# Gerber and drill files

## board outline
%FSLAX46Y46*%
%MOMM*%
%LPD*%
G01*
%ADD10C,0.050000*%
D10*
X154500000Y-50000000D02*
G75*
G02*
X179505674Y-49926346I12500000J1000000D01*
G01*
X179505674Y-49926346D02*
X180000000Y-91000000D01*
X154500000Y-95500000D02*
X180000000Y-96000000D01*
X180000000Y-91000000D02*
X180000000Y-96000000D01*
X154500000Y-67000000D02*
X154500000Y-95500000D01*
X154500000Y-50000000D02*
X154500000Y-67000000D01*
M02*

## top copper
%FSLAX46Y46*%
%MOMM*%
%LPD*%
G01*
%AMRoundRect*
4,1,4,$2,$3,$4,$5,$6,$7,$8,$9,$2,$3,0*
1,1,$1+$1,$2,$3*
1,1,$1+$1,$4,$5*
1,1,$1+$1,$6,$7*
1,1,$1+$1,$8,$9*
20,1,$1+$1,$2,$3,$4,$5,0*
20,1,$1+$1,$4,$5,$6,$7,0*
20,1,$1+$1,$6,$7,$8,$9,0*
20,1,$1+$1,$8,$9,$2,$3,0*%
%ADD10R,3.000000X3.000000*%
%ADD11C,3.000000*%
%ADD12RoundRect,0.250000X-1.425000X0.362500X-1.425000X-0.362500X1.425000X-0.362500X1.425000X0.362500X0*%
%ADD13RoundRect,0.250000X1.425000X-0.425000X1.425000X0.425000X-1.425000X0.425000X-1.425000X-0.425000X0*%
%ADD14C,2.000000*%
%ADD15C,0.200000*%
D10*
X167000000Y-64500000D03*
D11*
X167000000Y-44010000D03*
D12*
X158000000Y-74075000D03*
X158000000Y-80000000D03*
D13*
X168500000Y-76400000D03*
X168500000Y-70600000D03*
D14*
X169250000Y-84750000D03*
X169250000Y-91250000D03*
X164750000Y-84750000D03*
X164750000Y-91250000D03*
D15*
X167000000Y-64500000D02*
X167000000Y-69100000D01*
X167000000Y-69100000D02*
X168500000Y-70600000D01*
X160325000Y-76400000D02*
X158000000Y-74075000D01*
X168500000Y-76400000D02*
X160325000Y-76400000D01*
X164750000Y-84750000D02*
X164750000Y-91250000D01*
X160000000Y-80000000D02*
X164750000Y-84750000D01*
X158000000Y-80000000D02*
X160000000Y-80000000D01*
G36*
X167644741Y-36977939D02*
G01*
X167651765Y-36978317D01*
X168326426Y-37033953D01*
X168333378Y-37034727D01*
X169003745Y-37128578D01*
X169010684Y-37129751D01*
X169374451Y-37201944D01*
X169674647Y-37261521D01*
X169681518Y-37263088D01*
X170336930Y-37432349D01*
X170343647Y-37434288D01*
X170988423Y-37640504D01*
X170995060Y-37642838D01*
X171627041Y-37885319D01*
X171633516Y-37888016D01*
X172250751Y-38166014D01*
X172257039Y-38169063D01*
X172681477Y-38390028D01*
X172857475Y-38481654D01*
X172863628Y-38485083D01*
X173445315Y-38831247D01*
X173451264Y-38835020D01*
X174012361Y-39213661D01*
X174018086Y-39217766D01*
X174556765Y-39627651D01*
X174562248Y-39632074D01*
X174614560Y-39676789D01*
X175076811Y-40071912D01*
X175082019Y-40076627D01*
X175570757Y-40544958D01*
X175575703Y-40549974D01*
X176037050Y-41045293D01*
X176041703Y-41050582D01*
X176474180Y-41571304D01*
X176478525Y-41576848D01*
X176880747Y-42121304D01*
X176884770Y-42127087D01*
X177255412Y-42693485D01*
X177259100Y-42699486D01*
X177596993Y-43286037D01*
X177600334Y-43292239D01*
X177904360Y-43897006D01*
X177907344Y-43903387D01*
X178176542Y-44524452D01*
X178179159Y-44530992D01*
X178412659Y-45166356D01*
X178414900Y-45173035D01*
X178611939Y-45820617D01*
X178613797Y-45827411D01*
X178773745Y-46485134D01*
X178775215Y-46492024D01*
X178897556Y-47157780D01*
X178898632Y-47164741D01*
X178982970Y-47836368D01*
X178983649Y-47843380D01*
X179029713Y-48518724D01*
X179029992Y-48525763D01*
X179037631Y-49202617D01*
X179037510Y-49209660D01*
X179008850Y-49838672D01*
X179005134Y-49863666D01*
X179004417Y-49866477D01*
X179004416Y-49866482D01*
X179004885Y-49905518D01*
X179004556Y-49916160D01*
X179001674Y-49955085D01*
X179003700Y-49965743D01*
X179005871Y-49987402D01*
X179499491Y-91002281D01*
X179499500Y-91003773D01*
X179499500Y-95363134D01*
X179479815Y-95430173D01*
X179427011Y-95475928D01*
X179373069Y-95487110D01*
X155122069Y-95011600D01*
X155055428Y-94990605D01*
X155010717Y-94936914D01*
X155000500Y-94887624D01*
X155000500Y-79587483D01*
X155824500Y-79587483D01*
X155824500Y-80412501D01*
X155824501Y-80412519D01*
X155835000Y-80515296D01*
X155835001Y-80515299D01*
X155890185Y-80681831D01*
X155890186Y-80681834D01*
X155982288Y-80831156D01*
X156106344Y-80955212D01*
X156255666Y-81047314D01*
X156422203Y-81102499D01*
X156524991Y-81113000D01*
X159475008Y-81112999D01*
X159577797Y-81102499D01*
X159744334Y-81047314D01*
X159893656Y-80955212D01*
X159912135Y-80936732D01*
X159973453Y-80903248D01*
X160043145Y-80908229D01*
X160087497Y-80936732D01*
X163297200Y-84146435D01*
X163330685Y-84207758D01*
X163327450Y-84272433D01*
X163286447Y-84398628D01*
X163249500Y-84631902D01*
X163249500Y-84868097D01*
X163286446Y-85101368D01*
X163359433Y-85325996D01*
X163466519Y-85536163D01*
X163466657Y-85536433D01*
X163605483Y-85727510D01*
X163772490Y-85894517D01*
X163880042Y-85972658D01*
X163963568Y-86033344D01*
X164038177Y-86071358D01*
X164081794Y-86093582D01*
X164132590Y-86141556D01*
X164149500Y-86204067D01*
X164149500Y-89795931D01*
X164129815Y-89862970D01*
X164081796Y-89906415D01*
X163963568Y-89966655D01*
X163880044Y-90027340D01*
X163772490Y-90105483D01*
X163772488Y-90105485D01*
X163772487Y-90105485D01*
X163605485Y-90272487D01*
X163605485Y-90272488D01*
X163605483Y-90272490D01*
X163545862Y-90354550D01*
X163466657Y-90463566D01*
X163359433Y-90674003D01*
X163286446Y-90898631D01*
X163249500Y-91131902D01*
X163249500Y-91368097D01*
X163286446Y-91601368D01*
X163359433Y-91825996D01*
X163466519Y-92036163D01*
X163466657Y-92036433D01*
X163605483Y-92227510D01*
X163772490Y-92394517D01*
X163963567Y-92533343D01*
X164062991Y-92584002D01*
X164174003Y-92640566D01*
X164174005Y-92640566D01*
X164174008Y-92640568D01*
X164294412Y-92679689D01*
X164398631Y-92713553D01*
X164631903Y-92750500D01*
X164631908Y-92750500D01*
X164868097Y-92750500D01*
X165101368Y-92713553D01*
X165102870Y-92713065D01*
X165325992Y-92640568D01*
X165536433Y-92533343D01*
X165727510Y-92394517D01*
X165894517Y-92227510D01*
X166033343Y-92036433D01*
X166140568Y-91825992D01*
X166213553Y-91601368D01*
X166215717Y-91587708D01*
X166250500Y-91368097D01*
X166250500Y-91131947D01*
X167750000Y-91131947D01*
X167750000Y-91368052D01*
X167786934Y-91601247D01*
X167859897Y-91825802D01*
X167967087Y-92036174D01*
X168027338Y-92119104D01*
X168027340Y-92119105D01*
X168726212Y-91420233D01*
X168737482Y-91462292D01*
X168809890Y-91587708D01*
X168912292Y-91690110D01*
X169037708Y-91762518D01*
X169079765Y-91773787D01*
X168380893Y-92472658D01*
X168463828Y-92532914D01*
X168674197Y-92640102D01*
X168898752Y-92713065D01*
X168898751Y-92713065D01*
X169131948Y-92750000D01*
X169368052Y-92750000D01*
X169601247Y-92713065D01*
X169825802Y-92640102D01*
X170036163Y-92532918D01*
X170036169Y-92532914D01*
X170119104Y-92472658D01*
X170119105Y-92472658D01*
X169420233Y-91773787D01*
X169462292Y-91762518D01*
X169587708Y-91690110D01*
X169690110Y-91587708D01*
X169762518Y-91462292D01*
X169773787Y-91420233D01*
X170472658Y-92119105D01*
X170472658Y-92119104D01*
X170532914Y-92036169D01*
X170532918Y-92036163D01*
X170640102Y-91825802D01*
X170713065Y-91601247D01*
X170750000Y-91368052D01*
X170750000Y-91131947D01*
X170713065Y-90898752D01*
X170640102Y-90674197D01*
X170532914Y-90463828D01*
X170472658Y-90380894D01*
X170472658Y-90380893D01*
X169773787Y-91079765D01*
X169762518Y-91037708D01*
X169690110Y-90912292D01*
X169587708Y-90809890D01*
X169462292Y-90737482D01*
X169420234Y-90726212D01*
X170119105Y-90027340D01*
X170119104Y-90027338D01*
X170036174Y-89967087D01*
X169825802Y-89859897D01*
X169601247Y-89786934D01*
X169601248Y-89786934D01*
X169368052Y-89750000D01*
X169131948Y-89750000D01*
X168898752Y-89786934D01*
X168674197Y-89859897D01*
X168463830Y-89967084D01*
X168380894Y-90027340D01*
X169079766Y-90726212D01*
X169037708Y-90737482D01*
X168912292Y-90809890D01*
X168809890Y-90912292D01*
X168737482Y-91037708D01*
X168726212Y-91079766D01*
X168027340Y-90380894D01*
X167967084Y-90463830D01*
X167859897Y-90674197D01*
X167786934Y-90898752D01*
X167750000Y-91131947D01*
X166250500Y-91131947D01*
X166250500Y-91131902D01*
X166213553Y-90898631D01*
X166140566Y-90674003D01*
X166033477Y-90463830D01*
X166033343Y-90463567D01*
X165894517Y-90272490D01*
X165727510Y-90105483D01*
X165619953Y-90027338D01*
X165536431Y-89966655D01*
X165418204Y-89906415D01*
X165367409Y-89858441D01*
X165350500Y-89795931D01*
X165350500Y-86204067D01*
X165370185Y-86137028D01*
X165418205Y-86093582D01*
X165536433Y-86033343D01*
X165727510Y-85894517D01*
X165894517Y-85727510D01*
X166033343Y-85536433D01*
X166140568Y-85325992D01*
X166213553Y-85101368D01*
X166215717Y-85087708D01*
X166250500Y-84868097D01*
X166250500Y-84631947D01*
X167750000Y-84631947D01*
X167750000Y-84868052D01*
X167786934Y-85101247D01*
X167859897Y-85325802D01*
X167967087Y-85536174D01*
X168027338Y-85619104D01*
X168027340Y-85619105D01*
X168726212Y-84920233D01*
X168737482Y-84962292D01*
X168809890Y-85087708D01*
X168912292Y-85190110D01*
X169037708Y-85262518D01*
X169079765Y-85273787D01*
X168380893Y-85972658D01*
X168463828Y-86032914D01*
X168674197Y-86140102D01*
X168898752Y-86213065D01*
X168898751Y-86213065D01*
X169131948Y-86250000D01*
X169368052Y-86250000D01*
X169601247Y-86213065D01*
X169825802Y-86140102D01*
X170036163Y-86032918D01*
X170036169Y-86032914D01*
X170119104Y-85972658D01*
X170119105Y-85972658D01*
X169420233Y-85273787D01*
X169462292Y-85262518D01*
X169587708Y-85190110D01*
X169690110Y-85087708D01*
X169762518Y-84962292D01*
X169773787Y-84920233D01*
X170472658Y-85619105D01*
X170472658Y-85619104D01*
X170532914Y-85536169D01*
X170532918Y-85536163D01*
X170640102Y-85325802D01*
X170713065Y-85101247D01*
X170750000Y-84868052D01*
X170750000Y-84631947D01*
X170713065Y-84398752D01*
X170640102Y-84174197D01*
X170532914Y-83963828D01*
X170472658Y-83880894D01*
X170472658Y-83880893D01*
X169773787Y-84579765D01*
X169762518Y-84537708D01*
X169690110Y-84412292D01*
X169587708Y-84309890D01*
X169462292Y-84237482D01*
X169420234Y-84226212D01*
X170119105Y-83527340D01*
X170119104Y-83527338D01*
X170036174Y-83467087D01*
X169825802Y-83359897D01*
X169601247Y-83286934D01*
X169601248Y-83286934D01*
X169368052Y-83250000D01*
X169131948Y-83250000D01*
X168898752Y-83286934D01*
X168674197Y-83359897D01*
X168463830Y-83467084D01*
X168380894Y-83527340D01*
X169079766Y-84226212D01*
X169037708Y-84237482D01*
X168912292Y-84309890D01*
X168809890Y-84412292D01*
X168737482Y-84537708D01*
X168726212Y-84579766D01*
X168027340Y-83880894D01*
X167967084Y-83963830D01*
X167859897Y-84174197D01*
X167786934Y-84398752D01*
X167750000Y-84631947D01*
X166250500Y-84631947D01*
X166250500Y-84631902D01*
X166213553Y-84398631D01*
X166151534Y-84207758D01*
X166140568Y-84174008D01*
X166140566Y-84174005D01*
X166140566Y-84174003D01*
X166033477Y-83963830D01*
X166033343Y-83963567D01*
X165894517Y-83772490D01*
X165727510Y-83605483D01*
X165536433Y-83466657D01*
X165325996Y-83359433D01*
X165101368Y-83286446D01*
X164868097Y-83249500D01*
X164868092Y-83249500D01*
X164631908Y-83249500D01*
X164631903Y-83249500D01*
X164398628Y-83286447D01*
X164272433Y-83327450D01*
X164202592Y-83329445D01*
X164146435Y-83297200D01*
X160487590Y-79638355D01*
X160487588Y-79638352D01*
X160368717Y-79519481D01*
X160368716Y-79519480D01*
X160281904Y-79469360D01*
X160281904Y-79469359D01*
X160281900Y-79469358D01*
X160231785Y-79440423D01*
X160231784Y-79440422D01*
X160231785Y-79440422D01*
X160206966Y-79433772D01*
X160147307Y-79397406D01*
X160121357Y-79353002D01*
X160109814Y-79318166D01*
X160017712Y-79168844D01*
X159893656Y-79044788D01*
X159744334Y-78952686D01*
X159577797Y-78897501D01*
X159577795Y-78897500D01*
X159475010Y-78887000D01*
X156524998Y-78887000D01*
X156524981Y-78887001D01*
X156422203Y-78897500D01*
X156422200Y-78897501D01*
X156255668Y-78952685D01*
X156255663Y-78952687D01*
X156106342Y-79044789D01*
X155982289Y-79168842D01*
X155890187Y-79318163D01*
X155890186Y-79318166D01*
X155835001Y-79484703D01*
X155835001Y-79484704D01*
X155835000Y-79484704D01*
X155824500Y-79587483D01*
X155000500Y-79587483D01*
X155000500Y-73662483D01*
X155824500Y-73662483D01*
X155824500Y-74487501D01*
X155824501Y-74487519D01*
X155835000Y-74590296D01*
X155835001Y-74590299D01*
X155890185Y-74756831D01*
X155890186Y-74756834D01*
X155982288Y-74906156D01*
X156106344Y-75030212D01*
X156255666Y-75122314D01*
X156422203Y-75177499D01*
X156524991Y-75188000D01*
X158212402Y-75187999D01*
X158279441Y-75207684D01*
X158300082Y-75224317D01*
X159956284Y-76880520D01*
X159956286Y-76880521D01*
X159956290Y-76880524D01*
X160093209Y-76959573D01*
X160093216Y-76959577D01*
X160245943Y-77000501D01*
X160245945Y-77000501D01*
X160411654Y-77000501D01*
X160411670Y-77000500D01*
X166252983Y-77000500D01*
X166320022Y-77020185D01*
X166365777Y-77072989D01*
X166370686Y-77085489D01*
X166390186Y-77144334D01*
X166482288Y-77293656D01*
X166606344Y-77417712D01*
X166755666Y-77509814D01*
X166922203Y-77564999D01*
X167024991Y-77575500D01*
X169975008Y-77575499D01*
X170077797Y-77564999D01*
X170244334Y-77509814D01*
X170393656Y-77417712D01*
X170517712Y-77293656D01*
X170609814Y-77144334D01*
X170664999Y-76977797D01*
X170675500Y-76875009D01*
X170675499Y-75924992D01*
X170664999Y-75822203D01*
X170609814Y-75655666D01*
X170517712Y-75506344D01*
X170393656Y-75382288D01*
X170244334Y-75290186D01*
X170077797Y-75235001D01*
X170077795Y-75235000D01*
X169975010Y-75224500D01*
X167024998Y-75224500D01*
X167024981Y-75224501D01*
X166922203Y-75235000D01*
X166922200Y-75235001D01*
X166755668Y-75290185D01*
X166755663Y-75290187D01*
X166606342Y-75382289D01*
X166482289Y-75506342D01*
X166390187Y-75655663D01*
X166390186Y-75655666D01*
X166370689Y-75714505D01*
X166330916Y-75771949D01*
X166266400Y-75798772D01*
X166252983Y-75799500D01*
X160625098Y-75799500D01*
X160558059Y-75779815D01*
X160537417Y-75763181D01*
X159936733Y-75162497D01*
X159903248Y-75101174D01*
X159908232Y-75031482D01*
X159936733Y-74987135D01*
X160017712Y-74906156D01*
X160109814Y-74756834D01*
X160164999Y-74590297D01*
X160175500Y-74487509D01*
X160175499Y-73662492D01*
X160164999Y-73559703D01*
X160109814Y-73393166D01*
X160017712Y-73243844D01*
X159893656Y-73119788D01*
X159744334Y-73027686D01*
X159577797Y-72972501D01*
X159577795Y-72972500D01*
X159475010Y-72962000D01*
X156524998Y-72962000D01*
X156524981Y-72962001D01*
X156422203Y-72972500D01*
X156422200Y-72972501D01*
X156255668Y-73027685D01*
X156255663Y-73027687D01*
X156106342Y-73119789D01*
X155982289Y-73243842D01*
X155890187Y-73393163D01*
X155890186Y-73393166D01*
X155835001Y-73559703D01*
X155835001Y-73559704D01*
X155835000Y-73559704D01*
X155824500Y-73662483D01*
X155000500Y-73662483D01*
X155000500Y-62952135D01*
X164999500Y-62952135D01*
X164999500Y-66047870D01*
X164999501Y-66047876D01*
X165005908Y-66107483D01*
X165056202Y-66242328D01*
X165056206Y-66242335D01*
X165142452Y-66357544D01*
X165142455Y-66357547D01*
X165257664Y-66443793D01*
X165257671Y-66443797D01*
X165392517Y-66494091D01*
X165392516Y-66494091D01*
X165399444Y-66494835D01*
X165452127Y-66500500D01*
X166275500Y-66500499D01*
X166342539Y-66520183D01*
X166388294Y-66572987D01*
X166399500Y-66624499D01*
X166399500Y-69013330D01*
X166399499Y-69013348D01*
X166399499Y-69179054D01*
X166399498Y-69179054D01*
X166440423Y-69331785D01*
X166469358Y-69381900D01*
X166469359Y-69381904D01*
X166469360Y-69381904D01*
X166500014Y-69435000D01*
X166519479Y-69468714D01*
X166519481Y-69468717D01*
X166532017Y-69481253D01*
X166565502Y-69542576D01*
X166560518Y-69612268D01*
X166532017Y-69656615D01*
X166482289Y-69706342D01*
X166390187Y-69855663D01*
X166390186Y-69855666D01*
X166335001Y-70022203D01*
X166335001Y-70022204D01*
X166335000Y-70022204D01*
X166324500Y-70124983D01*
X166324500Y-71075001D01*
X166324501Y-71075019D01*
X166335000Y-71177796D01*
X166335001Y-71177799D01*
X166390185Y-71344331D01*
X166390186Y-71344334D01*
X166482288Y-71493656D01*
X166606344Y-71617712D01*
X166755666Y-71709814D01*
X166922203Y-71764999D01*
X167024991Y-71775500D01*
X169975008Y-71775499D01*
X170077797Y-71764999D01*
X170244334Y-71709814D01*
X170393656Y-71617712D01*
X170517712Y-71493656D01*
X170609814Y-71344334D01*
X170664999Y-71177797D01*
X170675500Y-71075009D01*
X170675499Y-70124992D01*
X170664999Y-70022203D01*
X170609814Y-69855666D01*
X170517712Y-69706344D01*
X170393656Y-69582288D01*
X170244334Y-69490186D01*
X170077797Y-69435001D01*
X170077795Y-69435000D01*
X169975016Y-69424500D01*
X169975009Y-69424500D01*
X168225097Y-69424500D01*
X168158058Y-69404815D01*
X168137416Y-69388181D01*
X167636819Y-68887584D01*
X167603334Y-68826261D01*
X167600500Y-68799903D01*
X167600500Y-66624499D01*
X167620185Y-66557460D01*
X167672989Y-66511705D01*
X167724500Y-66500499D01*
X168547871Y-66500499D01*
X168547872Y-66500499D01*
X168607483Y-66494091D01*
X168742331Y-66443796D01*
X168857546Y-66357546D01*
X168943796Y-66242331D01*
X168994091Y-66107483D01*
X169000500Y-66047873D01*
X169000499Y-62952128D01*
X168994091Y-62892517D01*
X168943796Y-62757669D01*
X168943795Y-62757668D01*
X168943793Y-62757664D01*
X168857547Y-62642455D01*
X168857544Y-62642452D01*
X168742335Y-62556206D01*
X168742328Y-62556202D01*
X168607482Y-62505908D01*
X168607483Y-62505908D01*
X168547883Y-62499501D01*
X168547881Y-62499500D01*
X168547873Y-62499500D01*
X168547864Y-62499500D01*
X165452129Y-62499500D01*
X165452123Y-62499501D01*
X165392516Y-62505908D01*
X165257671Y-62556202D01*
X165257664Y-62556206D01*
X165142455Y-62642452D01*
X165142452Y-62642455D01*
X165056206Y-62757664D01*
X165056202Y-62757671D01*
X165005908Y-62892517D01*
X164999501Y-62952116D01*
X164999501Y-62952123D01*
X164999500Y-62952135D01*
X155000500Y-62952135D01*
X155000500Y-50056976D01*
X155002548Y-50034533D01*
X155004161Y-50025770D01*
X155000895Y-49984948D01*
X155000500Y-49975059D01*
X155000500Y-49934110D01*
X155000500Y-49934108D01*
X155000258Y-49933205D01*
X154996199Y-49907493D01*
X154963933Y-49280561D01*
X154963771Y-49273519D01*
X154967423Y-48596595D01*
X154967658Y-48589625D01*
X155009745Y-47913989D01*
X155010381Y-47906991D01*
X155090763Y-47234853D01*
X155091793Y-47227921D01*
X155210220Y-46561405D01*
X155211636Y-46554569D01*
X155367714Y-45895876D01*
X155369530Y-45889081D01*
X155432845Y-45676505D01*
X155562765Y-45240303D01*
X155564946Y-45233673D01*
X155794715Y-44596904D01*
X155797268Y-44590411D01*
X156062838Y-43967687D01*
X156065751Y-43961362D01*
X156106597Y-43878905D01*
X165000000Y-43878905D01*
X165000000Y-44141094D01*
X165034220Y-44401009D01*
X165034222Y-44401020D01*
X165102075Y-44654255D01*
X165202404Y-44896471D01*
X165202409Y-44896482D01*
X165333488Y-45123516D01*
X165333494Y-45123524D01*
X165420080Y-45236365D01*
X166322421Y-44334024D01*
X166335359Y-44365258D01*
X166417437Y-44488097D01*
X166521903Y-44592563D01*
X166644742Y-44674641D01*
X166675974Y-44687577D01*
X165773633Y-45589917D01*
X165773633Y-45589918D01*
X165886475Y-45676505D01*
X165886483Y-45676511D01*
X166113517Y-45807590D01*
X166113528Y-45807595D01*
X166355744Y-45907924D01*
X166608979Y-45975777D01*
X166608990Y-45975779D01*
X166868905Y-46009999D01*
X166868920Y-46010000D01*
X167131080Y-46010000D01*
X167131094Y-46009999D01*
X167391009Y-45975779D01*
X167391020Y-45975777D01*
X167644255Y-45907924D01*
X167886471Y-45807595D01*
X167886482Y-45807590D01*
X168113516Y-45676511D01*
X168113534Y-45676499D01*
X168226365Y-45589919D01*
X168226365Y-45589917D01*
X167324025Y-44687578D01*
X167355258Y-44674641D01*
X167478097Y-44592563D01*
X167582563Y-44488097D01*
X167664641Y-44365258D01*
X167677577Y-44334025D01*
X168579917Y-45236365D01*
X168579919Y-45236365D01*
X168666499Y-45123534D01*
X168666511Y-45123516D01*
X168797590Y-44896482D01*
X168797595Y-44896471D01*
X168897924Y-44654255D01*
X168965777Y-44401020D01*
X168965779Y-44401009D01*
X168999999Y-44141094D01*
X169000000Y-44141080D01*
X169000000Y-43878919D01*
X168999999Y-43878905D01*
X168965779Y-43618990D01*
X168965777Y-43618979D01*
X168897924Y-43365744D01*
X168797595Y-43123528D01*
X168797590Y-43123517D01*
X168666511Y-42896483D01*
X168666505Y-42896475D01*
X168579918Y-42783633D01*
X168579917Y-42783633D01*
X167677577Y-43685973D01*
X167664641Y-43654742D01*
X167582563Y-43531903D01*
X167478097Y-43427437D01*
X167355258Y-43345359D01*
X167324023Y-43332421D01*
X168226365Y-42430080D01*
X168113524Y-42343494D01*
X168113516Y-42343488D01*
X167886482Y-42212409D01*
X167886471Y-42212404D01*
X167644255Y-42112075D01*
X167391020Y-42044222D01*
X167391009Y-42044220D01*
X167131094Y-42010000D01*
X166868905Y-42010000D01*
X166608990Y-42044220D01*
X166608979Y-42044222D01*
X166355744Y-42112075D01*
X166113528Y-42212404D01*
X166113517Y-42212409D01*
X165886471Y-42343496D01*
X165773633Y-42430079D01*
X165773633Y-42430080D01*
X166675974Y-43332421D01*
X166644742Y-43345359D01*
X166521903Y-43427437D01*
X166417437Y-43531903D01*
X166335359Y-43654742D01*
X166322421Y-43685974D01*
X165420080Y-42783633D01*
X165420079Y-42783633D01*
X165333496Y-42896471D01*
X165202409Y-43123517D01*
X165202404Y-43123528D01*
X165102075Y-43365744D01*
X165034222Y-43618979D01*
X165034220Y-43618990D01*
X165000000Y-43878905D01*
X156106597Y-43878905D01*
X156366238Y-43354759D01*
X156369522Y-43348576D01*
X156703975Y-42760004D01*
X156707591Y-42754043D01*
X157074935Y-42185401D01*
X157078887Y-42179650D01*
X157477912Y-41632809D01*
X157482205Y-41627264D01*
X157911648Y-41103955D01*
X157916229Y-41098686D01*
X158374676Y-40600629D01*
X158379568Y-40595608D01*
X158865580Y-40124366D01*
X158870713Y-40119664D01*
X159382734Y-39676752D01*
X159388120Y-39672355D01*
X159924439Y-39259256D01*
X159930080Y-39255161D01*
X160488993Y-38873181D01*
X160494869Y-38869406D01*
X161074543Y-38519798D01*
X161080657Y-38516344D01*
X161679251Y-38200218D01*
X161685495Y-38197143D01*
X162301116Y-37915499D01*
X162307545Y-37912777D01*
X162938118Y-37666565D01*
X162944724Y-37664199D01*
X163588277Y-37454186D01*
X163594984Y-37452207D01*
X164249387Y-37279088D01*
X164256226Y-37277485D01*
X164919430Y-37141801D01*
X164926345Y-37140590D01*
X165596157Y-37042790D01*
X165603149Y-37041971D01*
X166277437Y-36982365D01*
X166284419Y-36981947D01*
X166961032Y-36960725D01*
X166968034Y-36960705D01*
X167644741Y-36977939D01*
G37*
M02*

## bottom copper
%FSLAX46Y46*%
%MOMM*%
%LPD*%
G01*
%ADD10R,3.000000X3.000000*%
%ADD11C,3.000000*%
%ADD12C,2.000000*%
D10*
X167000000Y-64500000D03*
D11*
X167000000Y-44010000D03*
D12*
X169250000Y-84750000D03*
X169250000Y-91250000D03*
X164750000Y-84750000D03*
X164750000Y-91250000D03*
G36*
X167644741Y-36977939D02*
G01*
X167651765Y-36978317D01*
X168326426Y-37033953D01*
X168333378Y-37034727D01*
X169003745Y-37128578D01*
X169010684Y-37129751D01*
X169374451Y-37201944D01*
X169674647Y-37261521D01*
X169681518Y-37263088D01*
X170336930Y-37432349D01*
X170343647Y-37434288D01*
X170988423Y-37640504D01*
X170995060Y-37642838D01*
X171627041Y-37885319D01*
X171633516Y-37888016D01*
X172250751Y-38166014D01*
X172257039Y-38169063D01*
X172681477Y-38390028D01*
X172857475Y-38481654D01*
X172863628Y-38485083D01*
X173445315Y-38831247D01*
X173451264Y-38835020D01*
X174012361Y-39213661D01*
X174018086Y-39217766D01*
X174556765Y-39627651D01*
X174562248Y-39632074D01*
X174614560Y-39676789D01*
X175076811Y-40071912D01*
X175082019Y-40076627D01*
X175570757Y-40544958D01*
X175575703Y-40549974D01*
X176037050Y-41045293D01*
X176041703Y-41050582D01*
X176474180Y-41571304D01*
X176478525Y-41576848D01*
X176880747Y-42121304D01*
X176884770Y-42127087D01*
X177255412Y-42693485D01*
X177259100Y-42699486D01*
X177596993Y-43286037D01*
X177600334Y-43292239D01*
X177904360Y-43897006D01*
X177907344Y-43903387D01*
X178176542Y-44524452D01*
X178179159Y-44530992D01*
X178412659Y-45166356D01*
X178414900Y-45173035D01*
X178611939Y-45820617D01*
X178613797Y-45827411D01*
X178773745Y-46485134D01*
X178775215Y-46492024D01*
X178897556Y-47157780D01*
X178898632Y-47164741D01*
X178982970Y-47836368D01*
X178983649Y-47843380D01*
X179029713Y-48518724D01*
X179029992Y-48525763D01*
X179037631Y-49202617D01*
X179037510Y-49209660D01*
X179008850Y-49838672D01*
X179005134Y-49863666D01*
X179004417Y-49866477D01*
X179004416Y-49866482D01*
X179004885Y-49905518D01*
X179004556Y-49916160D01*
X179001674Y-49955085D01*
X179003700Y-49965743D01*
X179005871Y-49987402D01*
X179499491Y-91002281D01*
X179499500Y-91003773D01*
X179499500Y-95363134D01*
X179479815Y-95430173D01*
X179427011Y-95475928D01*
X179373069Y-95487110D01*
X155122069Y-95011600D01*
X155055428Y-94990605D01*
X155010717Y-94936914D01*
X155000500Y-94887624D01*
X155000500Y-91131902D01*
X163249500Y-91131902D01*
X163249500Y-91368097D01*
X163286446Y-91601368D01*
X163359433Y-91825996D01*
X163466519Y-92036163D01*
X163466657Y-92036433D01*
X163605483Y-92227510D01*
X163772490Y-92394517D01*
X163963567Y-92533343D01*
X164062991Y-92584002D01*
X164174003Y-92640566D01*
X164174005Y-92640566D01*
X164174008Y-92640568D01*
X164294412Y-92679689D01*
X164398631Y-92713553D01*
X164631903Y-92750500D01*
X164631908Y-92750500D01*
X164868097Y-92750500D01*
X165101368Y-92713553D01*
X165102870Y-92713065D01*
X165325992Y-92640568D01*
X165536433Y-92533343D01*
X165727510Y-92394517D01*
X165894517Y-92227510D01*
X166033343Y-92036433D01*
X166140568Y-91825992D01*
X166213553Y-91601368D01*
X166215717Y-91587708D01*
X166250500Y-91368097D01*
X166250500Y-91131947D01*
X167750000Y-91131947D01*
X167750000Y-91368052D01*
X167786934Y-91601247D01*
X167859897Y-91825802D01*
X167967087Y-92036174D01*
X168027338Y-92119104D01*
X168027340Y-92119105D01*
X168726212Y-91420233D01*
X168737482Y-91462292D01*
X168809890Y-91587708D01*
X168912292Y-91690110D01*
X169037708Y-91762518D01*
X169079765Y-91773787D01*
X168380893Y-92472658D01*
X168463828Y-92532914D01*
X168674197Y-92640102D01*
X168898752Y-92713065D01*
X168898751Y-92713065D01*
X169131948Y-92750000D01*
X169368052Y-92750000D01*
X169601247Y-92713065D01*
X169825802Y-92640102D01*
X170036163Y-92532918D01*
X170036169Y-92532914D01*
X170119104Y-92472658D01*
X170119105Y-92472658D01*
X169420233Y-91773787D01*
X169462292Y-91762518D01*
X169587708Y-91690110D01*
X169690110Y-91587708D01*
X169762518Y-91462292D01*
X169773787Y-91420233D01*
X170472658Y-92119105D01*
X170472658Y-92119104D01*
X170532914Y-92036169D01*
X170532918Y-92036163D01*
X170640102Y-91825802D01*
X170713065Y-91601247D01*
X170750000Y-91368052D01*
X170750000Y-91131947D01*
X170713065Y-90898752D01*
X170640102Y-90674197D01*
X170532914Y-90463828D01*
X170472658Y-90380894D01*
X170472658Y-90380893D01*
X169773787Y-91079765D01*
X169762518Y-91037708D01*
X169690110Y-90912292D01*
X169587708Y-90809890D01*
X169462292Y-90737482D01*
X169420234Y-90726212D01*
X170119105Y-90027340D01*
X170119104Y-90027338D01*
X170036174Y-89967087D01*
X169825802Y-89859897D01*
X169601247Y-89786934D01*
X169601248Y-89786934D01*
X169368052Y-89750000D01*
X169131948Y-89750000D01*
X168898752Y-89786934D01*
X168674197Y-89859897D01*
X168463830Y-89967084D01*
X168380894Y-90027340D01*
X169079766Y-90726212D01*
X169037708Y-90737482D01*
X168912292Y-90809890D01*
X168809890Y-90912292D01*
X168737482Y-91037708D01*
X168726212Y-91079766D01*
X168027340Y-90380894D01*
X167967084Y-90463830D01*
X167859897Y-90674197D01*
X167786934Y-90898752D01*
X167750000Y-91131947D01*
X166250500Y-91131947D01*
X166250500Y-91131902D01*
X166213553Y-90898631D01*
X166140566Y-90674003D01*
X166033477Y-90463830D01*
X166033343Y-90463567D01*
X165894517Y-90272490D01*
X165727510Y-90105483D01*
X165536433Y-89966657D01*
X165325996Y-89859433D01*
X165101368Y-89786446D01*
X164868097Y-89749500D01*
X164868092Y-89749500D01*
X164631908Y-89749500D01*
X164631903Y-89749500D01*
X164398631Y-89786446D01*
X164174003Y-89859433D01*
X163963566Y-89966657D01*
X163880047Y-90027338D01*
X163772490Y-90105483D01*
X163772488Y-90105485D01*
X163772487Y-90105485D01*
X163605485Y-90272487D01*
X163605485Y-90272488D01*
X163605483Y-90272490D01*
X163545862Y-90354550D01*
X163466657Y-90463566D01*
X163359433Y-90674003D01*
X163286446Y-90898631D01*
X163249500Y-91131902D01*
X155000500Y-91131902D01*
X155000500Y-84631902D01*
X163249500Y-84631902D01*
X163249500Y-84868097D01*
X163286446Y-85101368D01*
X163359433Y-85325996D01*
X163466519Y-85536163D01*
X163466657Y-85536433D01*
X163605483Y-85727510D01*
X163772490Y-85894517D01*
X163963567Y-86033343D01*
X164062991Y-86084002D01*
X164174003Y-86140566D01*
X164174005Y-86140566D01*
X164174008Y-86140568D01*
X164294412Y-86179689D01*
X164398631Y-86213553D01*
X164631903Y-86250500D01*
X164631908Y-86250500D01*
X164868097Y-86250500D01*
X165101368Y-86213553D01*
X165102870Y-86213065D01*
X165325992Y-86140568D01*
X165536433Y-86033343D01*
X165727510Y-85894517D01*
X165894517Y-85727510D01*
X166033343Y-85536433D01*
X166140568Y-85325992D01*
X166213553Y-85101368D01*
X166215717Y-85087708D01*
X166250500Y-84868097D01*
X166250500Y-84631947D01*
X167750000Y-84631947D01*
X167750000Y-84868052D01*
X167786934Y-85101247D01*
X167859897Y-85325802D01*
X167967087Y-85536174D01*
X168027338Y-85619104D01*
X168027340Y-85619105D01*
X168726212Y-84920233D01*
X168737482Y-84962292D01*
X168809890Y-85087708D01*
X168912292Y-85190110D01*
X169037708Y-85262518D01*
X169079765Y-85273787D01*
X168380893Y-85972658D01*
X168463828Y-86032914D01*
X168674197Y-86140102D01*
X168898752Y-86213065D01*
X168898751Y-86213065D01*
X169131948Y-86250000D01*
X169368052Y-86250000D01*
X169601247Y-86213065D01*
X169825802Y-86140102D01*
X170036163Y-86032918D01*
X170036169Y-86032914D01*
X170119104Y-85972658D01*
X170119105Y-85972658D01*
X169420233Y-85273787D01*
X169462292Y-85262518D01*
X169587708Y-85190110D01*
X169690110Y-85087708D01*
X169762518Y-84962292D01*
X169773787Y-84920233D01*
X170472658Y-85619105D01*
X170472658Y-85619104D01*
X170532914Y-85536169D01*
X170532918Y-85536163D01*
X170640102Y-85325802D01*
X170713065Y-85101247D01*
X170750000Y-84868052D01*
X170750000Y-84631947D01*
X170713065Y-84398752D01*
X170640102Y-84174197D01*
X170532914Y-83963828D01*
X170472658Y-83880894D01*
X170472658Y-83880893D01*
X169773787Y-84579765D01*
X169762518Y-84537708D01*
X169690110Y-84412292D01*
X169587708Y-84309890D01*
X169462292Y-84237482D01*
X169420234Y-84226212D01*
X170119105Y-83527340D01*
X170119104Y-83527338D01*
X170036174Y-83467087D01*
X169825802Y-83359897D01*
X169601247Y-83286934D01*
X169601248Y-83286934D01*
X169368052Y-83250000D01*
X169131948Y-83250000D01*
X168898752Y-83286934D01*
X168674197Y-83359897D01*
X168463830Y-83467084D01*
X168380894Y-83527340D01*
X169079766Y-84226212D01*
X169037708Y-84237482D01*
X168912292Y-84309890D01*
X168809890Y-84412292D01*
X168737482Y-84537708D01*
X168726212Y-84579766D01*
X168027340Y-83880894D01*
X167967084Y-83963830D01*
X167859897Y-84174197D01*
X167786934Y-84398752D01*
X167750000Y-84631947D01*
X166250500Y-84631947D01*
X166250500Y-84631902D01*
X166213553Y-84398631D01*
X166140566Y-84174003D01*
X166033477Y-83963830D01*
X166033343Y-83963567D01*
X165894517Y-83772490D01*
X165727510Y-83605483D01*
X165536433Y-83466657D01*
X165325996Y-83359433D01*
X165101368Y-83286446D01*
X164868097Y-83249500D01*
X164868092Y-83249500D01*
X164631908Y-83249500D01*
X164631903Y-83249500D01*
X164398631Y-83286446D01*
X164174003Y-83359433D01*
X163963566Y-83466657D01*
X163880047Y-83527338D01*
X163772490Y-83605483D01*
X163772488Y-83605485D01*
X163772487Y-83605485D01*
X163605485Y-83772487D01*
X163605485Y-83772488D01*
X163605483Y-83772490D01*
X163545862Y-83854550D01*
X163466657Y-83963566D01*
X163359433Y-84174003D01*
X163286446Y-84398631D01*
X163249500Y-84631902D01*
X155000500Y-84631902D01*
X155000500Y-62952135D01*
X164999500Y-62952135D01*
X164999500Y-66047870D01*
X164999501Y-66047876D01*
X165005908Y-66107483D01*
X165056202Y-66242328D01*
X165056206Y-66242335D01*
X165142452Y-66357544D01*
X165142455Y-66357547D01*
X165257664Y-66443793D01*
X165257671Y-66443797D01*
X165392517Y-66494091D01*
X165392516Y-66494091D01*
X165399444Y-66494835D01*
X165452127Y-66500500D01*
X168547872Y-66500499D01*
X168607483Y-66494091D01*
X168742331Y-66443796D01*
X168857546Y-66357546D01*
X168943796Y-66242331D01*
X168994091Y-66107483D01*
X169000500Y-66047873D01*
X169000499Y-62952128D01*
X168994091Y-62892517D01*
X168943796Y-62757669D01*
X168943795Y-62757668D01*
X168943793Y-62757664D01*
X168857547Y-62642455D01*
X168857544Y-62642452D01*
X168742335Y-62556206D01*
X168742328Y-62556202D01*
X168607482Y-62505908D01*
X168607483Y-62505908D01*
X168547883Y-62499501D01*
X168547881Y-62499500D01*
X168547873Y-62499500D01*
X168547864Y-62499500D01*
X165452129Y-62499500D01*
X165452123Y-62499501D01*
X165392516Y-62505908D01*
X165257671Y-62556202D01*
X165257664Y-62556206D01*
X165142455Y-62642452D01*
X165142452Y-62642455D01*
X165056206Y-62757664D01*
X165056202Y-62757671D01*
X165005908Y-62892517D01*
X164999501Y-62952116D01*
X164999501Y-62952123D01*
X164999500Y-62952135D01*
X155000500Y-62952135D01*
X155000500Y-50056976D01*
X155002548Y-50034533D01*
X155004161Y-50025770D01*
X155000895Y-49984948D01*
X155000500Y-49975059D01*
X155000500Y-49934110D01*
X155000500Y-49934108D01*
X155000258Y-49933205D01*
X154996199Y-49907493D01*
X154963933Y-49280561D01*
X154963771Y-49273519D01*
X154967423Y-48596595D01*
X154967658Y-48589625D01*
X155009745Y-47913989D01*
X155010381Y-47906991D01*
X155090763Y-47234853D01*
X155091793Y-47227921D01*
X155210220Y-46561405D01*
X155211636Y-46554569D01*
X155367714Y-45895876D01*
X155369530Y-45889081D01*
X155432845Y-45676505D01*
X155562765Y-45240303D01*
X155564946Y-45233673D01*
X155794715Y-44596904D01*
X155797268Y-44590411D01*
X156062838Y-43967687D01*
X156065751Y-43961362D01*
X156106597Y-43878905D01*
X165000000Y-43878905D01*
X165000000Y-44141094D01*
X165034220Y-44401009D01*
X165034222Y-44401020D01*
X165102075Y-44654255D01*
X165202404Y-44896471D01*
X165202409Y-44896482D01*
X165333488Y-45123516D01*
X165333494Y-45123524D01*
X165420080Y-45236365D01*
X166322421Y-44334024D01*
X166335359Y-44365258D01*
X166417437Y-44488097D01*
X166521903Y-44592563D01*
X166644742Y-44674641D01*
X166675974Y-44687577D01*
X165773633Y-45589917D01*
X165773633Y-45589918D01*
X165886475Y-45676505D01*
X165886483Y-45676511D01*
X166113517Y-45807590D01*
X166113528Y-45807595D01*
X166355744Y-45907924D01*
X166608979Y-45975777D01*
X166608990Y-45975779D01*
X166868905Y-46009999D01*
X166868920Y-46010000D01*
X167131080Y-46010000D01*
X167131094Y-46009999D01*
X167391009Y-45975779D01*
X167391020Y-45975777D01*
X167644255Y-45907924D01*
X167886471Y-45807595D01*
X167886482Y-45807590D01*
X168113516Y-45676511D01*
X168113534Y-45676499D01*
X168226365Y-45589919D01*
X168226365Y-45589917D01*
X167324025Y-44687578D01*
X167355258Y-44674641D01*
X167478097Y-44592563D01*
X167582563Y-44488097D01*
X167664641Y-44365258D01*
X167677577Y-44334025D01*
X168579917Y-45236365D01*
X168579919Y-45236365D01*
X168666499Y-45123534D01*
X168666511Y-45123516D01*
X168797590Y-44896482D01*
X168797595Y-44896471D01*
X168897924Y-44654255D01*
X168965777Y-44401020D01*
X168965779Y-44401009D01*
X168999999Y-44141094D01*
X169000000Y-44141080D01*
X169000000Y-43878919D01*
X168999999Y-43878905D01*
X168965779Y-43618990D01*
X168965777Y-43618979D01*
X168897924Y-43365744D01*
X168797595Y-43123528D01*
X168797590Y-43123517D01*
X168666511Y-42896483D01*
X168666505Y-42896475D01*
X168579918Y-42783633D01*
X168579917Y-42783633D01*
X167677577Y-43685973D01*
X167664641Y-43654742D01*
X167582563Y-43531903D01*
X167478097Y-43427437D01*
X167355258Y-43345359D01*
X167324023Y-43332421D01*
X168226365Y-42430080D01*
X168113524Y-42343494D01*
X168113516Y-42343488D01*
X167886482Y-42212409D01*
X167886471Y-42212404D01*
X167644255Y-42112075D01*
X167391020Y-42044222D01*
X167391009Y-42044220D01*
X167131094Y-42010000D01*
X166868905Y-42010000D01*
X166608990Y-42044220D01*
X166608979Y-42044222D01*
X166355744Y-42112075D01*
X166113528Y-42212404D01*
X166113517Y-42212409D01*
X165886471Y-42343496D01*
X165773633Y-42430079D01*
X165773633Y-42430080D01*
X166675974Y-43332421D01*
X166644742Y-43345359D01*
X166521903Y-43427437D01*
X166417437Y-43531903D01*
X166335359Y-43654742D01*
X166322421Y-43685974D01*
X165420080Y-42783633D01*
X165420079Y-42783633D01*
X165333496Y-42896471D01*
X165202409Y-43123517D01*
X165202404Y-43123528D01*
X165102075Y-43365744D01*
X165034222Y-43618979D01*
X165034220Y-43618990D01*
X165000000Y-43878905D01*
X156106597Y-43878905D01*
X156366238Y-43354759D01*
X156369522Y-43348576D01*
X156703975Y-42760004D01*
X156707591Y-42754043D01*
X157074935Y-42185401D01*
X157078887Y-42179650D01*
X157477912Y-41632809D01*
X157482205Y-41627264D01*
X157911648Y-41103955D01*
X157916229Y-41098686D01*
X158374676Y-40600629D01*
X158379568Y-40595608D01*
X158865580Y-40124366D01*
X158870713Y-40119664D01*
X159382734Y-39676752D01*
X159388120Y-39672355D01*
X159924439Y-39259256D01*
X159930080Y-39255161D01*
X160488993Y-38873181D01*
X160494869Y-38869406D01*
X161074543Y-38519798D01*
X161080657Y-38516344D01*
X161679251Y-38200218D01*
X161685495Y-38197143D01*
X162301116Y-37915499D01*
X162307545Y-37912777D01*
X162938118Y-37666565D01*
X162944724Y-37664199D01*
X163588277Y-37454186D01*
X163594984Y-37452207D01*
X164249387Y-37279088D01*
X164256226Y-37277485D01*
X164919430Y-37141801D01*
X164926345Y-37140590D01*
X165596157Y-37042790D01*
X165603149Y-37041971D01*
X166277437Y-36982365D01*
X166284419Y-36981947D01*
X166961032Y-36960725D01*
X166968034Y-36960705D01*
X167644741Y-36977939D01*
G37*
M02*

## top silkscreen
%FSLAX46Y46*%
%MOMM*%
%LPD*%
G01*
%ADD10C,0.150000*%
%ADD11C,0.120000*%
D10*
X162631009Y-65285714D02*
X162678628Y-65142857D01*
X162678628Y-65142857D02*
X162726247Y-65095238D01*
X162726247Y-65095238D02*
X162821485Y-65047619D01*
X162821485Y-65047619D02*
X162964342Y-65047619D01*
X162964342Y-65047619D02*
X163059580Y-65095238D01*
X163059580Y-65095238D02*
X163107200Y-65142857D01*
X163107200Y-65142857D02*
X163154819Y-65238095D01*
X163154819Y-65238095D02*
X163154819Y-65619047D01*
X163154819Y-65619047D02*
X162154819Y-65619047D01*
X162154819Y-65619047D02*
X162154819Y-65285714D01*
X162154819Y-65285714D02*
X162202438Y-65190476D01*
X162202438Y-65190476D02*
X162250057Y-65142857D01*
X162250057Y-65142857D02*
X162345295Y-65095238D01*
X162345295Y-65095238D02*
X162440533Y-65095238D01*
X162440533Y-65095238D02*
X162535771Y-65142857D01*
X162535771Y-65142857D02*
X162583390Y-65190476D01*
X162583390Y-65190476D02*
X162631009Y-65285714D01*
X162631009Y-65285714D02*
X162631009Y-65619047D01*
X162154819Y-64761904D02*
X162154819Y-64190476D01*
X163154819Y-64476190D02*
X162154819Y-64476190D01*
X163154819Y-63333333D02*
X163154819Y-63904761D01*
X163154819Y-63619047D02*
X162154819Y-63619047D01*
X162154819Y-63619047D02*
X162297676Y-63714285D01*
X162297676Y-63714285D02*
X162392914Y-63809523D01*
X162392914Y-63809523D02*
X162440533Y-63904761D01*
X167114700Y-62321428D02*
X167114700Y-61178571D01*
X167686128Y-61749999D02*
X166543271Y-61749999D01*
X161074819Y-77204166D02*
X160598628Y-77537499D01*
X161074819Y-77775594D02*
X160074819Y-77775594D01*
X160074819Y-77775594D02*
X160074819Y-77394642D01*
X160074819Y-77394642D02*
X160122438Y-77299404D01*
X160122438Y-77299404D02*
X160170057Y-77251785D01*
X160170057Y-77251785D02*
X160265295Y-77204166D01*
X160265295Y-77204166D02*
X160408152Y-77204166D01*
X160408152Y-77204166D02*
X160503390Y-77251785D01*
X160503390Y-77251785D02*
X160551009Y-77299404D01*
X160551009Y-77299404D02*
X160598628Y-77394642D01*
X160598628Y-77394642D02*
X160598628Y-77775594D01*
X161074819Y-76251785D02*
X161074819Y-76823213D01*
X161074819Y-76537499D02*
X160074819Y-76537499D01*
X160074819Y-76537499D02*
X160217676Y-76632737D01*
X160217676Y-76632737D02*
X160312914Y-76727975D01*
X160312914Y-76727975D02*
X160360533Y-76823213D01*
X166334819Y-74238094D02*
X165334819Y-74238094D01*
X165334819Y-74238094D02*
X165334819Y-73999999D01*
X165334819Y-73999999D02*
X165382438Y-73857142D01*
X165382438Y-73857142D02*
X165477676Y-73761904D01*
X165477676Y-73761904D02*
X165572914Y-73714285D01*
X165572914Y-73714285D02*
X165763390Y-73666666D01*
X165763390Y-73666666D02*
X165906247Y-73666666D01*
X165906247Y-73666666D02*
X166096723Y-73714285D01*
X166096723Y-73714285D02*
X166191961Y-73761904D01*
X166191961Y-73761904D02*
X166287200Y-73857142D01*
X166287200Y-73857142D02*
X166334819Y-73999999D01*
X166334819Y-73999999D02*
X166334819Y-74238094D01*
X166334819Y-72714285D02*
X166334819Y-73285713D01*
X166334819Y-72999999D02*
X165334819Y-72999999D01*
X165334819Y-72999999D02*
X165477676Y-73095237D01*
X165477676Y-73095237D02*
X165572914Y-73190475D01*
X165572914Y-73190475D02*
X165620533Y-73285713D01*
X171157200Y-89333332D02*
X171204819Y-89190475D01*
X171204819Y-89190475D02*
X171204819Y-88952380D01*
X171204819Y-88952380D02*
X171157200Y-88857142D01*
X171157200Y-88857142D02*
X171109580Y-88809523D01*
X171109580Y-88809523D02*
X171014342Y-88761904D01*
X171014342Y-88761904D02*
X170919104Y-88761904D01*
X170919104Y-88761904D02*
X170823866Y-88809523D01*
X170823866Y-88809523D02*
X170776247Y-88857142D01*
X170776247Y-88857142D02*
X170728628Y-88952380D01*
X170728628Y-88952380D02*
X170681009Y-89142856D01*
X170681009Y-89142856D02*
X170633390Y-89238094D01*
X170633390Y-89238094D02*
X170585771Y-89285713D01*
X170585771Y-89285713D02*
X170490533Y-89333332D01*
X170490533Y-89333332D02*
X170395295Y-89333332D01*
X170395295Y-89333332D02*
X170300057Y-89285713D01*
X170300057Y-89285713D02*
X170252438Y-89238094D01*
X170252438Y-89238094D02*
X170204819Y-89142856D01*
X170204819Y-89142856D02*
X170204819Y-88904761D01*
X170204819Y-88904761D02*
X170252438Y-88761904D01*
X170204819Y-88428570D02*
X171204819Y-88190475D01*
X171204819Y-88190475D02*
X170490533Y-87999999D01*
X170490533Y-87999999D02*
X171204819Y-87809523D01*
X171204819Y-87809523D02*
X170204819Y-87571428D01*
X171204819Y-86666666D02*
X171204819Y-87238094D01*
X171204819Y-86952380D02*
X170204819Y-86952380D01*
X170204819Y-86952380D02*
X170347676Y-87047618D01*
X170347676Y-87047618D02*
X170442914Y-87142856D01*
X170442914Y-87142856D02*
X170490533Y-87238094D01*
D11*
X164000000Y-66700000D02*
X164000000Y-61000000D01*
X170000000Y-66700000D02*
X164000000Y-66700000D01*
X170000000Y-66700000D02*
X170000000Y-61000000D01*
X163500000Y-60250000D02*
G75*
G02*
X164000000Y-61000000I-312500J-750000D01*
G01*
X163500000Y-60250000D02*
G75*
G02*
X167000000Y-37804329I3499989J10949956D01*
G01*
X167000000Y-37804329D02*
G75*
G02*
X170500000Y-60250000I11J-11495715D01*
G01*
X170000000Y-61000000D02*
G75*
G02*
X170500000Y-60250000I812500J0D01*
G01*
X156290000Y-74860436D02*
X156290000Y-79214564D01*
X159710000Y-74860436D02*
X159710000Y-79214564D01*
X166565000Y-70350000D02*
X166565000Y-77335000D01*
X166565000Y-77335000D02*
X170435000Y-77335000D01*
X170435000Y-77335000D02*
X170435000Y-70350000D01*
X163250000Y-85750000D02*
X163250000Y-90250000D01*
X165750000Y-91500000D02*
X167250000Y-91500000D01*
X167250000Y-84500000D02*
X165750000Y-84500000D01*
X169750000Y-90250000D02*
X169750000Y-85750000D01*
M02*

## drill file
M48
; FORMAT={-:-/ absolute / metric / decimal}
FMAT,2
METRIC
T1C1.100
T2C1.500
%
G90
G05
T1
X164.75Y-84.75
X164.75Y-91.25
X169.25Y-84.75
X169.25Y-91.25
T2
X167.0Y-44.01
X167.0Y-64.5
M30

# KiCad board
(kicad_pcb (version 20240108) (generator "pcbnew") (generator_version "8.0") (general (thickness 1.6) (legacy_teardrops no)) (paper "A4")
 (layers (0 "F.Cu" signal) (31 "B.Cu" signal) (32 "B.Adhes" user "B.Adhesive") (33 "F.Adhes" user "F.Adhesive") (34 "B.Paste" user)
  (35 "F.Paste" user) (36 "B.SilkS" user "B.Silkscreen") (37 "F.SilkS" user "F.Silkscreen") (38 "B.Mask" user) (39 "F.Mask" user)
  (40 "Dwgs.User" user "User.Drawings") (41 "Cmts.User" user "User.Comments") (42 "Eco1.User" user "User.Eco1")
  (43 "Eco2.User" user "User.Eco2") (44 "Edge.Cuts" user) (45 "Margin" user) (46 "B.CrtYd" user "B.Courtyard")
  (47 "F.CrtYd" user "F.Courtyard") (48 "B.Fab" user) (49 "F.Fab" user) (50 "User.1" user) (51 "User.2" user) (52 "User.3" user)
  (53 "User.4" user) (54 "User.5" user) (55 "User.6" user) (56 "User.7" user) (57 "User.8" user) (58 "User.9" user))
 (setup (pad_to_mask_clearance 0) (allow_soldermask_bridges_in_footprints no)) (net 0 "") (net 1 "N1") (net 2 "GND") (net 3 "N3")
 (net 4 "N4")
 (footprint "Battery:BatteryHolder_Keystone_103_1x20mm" (layer "F.Cu") (at 167 64.5 90)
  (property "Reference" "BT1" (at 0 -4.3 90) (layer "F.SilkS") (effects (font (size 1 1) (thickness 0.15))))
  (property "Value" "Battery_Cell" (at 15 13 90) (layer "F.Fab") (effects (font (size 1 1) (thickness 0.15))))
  (fp_line (start -2.2 -3) (end 3.5 -3) (stroke (width 0.12) (type solid)) (layer "F.SilkS"))
  (fp_line (start -2.2 3) (end -2.2 -3) (stroke (width 0.12) (type solid)) (layer "F.SilkS"))
  (fp_line (start -2.2 3) (end 3.5 3) (stroke (width 0.12) (type solid)) (layer "F.SilkS"))
  (fp_arc (start 4.25 -3.5) (mid 3.950694 -3.136459) (end 3.5 -3) (stroke (width 0.12) (type solid)) (layer "F.SilkS"))
  (fp_arc (start 4.25 -3.5) (mid 16.971103 -11.358466) (end 26.695671 0) (stroke (width 0.12) (type solid)) (layer "F.SilkS"))
  (fp_arc (start 26.695671 0) (mid 16.971103 11.358466) (end 4.25 3.5) (stroke (width 0.12) (type solid)) (layer "F.SilkS"))
  (fp_arc (start 3.5 3) (mid 3.950694 3.136459) (end 4.25 3.5) (stroke (width 0.12) (type solid)) (layer "F.SilkS"))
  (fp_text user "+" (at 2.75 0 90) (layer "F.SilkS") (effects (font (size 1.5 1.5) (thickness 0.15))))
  (pad "1" thru_hole rect (at 0 0 90) (size 3 3) (drill 1.5) (layers "*.Cu" "*.Mask") (remove_unused_layers no) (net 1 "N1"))
  (pad "2" thru_hole circle (at 20.49 0 90) (size 3 3) (drill 1.5) (layers "*.Cu" "*.Mask") (remove_unused_layers no) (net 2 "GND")))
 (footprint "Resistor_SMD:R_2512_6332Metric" (layer "F.Cu") (at 158 77.0375 -90)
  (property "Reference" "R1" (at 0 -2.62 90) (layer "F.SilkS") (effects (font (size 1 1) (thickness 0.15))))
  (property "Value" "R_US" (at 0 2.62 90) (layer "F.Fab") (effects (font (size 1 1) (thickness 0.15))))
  (fp_line (start -2.177064 1.71) (end 2.177064 1.71) (stroke (width 0.12) (type solid)) (layer "F.SilkS"))
  (fp_line (start -2.177064 -1.71) (end 2.177064 -1.71) (stroke (width 0.12) (type solid)) (layer "F.SilkS"))
  (pad "1" smd roundrect (at -2.9625 0 270) (size 1.225 3.35) (layers "F.Cu" "F.Paste" "F.Mask") (roundrect_rratio 0.204082) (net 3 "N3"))
  (pad "2" smd roundrect (at 2.9625 0 270) (size 1.225 3.35) (layers "F.Cu" "F.Paste" "F.Mask") (roundrect_rratio 0.204082) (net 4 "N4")))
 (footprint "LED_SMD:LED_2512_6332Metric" (layer "F.Cu") (at 168.5 73.5 90)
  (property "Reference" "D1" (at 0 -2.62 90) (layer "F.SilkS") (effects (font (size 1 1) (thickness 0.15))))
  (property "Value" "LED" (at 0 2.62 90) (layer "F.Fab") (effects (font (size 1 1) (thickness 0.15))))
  (fp_line (start 3.15 -1.935) (end -3.835 -1.935) (stroke (width 0.12) (type solid)) (layer "F.SilkS"))
  (fp_line (start -3.835 -1.935) (end -3.835 1.935) (stroke (width 0.12) (type solid)) (layer "F.SilkS"))
  (fp_line (start -3.835 1.935) (end 3.15 1.935) (stroke (width 0.12) (type solid)) (layer "F.SilkS"))
  (pad "1" smd roundrect (at -2.9 0 90) (size 1.35 3.35) (layers "F.Cu" "F.Paste" "F.Mask") (roundrect_rratio 0.185185) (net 3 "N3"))
  (pad "2" smd roundrect (at 2.9 0 90) (size 1.35 3.35) (layers "F.Cu" "F.Paste" "F.Mask") (roundrect_rratio 0.185185) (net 1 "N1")))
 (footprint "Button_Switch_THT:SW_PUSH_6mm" (layer "F.Cu") (at 168.75 84.75 -90)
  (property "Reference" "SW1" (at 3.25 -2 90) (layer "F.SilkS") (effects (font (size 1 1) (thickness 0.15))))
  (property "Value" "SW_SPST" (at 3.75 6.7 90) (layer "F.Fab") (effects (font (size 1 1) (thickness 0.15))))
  (fp_line (start 1 5.5) (end 5.5 5.5) (stroke (width 0.12) (type solid)) (layer "F.SilkS"))
  (fp_line (start 6.75 3) (end 6.75 1.5) (stroke (width 0.12) (type solid)) (layer "F.SilkS"))
  (fp_line (start -0.25 1.5) (end -0.25 3) (stroke (width 0.12) (type solid)) (layer "F.SilkS"))
  (fp_line (start 5.5 -1) (end 1 -1) (stroke (width 0.12) (type solid)) (layer "F.SilkS"))
  (pad "1" thru_hole circle (at 0 -0.5) (size 2 2) (drill 1.1) (layers "*.Cu" "*.Mask") (remove_unused_layers no) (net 2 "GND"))
  (pad "1" thru_hole circle (at 6.5 -0.5) (size 2 2) (drill 1.1) (layers "*.Cu" "*.Mask") (remove_unused_layers no) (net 2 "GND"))
  (pad "2" thru_hole circle (at 0 4) (size 2 2) (drill 1.1) (layers "*.Cu" "*.Mask") (remove_unused_layers no) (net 4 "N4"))
  (pad "2" thru_hole circle (at 6.5 4) (size 2 2) (drill 1.1) (layers "*.Cu" "*.Mask") (remove_unused_layers no) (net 4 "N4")))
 (gr_arc (start 154.5 50) (mid 166.963064 36.460118) (end 179.505674 49.926346) (stroke (width 0.05) (type default)) (layer "Edge.Cuts"))
 (gr_line (start 179.505674 49.926346) (end 180 91) (stroke (width 0.05) (type default)) (layer "Edge.Cuts"))
 (gr_line (start 154.5 95.5) (end 180 96) (stroke (width 0.05) (type default)) (layer "Edge.Cuts"))
 (gr_line (start 180 91) (end 180 96) (stroke (width 0.05) (type default)) (layer "Edge.Cuts"))
 (gr_line (start 154.5 67) (end 154.5 95.5) (stroke (width 0.05) (type default)) (layer "Edge.Cuts"))
 (gr_line (start 154.5 50) (end 154.5 67) (stroke (width 0.05) (type default)) (layer "Edge.Cuts"))
 (segment (start 167 64.5) (end 167 69.1) (width 0.2) (layer "F.Cu") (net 1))
 (segment (start 167 69.1) (end 168.5 70.6) (width 0.2) (layer "F.Cu") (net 1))
 (segment (start 160.325 76.4) (end 158 74.075) (width 0.2) (layer "F.Cu") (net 3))
 (segment (start 168.5 76.4) (end 160.325 76.4) (width 0.2) (layer "F.Cu") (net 3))
 (segment (start 164.75 84.75) (end 164.75 91.25) (width 0.2) (layer "F.Cu") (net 4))
 (segment (start 160 80) (end 164.75 84.75) (width 0.2) (layer "F.Cu") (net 4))
 (segment (start 158 80) (end 160 80) (width 0.2) (layer "F.Cu") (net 4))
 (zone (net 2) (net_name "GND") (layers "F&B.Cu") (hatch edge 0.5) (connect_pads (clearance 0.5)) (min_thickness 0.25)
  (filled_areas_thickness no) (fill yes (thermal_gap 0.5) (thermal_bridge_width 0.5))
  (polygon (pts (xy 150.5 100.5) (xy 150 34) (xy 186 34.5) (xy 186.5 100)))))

